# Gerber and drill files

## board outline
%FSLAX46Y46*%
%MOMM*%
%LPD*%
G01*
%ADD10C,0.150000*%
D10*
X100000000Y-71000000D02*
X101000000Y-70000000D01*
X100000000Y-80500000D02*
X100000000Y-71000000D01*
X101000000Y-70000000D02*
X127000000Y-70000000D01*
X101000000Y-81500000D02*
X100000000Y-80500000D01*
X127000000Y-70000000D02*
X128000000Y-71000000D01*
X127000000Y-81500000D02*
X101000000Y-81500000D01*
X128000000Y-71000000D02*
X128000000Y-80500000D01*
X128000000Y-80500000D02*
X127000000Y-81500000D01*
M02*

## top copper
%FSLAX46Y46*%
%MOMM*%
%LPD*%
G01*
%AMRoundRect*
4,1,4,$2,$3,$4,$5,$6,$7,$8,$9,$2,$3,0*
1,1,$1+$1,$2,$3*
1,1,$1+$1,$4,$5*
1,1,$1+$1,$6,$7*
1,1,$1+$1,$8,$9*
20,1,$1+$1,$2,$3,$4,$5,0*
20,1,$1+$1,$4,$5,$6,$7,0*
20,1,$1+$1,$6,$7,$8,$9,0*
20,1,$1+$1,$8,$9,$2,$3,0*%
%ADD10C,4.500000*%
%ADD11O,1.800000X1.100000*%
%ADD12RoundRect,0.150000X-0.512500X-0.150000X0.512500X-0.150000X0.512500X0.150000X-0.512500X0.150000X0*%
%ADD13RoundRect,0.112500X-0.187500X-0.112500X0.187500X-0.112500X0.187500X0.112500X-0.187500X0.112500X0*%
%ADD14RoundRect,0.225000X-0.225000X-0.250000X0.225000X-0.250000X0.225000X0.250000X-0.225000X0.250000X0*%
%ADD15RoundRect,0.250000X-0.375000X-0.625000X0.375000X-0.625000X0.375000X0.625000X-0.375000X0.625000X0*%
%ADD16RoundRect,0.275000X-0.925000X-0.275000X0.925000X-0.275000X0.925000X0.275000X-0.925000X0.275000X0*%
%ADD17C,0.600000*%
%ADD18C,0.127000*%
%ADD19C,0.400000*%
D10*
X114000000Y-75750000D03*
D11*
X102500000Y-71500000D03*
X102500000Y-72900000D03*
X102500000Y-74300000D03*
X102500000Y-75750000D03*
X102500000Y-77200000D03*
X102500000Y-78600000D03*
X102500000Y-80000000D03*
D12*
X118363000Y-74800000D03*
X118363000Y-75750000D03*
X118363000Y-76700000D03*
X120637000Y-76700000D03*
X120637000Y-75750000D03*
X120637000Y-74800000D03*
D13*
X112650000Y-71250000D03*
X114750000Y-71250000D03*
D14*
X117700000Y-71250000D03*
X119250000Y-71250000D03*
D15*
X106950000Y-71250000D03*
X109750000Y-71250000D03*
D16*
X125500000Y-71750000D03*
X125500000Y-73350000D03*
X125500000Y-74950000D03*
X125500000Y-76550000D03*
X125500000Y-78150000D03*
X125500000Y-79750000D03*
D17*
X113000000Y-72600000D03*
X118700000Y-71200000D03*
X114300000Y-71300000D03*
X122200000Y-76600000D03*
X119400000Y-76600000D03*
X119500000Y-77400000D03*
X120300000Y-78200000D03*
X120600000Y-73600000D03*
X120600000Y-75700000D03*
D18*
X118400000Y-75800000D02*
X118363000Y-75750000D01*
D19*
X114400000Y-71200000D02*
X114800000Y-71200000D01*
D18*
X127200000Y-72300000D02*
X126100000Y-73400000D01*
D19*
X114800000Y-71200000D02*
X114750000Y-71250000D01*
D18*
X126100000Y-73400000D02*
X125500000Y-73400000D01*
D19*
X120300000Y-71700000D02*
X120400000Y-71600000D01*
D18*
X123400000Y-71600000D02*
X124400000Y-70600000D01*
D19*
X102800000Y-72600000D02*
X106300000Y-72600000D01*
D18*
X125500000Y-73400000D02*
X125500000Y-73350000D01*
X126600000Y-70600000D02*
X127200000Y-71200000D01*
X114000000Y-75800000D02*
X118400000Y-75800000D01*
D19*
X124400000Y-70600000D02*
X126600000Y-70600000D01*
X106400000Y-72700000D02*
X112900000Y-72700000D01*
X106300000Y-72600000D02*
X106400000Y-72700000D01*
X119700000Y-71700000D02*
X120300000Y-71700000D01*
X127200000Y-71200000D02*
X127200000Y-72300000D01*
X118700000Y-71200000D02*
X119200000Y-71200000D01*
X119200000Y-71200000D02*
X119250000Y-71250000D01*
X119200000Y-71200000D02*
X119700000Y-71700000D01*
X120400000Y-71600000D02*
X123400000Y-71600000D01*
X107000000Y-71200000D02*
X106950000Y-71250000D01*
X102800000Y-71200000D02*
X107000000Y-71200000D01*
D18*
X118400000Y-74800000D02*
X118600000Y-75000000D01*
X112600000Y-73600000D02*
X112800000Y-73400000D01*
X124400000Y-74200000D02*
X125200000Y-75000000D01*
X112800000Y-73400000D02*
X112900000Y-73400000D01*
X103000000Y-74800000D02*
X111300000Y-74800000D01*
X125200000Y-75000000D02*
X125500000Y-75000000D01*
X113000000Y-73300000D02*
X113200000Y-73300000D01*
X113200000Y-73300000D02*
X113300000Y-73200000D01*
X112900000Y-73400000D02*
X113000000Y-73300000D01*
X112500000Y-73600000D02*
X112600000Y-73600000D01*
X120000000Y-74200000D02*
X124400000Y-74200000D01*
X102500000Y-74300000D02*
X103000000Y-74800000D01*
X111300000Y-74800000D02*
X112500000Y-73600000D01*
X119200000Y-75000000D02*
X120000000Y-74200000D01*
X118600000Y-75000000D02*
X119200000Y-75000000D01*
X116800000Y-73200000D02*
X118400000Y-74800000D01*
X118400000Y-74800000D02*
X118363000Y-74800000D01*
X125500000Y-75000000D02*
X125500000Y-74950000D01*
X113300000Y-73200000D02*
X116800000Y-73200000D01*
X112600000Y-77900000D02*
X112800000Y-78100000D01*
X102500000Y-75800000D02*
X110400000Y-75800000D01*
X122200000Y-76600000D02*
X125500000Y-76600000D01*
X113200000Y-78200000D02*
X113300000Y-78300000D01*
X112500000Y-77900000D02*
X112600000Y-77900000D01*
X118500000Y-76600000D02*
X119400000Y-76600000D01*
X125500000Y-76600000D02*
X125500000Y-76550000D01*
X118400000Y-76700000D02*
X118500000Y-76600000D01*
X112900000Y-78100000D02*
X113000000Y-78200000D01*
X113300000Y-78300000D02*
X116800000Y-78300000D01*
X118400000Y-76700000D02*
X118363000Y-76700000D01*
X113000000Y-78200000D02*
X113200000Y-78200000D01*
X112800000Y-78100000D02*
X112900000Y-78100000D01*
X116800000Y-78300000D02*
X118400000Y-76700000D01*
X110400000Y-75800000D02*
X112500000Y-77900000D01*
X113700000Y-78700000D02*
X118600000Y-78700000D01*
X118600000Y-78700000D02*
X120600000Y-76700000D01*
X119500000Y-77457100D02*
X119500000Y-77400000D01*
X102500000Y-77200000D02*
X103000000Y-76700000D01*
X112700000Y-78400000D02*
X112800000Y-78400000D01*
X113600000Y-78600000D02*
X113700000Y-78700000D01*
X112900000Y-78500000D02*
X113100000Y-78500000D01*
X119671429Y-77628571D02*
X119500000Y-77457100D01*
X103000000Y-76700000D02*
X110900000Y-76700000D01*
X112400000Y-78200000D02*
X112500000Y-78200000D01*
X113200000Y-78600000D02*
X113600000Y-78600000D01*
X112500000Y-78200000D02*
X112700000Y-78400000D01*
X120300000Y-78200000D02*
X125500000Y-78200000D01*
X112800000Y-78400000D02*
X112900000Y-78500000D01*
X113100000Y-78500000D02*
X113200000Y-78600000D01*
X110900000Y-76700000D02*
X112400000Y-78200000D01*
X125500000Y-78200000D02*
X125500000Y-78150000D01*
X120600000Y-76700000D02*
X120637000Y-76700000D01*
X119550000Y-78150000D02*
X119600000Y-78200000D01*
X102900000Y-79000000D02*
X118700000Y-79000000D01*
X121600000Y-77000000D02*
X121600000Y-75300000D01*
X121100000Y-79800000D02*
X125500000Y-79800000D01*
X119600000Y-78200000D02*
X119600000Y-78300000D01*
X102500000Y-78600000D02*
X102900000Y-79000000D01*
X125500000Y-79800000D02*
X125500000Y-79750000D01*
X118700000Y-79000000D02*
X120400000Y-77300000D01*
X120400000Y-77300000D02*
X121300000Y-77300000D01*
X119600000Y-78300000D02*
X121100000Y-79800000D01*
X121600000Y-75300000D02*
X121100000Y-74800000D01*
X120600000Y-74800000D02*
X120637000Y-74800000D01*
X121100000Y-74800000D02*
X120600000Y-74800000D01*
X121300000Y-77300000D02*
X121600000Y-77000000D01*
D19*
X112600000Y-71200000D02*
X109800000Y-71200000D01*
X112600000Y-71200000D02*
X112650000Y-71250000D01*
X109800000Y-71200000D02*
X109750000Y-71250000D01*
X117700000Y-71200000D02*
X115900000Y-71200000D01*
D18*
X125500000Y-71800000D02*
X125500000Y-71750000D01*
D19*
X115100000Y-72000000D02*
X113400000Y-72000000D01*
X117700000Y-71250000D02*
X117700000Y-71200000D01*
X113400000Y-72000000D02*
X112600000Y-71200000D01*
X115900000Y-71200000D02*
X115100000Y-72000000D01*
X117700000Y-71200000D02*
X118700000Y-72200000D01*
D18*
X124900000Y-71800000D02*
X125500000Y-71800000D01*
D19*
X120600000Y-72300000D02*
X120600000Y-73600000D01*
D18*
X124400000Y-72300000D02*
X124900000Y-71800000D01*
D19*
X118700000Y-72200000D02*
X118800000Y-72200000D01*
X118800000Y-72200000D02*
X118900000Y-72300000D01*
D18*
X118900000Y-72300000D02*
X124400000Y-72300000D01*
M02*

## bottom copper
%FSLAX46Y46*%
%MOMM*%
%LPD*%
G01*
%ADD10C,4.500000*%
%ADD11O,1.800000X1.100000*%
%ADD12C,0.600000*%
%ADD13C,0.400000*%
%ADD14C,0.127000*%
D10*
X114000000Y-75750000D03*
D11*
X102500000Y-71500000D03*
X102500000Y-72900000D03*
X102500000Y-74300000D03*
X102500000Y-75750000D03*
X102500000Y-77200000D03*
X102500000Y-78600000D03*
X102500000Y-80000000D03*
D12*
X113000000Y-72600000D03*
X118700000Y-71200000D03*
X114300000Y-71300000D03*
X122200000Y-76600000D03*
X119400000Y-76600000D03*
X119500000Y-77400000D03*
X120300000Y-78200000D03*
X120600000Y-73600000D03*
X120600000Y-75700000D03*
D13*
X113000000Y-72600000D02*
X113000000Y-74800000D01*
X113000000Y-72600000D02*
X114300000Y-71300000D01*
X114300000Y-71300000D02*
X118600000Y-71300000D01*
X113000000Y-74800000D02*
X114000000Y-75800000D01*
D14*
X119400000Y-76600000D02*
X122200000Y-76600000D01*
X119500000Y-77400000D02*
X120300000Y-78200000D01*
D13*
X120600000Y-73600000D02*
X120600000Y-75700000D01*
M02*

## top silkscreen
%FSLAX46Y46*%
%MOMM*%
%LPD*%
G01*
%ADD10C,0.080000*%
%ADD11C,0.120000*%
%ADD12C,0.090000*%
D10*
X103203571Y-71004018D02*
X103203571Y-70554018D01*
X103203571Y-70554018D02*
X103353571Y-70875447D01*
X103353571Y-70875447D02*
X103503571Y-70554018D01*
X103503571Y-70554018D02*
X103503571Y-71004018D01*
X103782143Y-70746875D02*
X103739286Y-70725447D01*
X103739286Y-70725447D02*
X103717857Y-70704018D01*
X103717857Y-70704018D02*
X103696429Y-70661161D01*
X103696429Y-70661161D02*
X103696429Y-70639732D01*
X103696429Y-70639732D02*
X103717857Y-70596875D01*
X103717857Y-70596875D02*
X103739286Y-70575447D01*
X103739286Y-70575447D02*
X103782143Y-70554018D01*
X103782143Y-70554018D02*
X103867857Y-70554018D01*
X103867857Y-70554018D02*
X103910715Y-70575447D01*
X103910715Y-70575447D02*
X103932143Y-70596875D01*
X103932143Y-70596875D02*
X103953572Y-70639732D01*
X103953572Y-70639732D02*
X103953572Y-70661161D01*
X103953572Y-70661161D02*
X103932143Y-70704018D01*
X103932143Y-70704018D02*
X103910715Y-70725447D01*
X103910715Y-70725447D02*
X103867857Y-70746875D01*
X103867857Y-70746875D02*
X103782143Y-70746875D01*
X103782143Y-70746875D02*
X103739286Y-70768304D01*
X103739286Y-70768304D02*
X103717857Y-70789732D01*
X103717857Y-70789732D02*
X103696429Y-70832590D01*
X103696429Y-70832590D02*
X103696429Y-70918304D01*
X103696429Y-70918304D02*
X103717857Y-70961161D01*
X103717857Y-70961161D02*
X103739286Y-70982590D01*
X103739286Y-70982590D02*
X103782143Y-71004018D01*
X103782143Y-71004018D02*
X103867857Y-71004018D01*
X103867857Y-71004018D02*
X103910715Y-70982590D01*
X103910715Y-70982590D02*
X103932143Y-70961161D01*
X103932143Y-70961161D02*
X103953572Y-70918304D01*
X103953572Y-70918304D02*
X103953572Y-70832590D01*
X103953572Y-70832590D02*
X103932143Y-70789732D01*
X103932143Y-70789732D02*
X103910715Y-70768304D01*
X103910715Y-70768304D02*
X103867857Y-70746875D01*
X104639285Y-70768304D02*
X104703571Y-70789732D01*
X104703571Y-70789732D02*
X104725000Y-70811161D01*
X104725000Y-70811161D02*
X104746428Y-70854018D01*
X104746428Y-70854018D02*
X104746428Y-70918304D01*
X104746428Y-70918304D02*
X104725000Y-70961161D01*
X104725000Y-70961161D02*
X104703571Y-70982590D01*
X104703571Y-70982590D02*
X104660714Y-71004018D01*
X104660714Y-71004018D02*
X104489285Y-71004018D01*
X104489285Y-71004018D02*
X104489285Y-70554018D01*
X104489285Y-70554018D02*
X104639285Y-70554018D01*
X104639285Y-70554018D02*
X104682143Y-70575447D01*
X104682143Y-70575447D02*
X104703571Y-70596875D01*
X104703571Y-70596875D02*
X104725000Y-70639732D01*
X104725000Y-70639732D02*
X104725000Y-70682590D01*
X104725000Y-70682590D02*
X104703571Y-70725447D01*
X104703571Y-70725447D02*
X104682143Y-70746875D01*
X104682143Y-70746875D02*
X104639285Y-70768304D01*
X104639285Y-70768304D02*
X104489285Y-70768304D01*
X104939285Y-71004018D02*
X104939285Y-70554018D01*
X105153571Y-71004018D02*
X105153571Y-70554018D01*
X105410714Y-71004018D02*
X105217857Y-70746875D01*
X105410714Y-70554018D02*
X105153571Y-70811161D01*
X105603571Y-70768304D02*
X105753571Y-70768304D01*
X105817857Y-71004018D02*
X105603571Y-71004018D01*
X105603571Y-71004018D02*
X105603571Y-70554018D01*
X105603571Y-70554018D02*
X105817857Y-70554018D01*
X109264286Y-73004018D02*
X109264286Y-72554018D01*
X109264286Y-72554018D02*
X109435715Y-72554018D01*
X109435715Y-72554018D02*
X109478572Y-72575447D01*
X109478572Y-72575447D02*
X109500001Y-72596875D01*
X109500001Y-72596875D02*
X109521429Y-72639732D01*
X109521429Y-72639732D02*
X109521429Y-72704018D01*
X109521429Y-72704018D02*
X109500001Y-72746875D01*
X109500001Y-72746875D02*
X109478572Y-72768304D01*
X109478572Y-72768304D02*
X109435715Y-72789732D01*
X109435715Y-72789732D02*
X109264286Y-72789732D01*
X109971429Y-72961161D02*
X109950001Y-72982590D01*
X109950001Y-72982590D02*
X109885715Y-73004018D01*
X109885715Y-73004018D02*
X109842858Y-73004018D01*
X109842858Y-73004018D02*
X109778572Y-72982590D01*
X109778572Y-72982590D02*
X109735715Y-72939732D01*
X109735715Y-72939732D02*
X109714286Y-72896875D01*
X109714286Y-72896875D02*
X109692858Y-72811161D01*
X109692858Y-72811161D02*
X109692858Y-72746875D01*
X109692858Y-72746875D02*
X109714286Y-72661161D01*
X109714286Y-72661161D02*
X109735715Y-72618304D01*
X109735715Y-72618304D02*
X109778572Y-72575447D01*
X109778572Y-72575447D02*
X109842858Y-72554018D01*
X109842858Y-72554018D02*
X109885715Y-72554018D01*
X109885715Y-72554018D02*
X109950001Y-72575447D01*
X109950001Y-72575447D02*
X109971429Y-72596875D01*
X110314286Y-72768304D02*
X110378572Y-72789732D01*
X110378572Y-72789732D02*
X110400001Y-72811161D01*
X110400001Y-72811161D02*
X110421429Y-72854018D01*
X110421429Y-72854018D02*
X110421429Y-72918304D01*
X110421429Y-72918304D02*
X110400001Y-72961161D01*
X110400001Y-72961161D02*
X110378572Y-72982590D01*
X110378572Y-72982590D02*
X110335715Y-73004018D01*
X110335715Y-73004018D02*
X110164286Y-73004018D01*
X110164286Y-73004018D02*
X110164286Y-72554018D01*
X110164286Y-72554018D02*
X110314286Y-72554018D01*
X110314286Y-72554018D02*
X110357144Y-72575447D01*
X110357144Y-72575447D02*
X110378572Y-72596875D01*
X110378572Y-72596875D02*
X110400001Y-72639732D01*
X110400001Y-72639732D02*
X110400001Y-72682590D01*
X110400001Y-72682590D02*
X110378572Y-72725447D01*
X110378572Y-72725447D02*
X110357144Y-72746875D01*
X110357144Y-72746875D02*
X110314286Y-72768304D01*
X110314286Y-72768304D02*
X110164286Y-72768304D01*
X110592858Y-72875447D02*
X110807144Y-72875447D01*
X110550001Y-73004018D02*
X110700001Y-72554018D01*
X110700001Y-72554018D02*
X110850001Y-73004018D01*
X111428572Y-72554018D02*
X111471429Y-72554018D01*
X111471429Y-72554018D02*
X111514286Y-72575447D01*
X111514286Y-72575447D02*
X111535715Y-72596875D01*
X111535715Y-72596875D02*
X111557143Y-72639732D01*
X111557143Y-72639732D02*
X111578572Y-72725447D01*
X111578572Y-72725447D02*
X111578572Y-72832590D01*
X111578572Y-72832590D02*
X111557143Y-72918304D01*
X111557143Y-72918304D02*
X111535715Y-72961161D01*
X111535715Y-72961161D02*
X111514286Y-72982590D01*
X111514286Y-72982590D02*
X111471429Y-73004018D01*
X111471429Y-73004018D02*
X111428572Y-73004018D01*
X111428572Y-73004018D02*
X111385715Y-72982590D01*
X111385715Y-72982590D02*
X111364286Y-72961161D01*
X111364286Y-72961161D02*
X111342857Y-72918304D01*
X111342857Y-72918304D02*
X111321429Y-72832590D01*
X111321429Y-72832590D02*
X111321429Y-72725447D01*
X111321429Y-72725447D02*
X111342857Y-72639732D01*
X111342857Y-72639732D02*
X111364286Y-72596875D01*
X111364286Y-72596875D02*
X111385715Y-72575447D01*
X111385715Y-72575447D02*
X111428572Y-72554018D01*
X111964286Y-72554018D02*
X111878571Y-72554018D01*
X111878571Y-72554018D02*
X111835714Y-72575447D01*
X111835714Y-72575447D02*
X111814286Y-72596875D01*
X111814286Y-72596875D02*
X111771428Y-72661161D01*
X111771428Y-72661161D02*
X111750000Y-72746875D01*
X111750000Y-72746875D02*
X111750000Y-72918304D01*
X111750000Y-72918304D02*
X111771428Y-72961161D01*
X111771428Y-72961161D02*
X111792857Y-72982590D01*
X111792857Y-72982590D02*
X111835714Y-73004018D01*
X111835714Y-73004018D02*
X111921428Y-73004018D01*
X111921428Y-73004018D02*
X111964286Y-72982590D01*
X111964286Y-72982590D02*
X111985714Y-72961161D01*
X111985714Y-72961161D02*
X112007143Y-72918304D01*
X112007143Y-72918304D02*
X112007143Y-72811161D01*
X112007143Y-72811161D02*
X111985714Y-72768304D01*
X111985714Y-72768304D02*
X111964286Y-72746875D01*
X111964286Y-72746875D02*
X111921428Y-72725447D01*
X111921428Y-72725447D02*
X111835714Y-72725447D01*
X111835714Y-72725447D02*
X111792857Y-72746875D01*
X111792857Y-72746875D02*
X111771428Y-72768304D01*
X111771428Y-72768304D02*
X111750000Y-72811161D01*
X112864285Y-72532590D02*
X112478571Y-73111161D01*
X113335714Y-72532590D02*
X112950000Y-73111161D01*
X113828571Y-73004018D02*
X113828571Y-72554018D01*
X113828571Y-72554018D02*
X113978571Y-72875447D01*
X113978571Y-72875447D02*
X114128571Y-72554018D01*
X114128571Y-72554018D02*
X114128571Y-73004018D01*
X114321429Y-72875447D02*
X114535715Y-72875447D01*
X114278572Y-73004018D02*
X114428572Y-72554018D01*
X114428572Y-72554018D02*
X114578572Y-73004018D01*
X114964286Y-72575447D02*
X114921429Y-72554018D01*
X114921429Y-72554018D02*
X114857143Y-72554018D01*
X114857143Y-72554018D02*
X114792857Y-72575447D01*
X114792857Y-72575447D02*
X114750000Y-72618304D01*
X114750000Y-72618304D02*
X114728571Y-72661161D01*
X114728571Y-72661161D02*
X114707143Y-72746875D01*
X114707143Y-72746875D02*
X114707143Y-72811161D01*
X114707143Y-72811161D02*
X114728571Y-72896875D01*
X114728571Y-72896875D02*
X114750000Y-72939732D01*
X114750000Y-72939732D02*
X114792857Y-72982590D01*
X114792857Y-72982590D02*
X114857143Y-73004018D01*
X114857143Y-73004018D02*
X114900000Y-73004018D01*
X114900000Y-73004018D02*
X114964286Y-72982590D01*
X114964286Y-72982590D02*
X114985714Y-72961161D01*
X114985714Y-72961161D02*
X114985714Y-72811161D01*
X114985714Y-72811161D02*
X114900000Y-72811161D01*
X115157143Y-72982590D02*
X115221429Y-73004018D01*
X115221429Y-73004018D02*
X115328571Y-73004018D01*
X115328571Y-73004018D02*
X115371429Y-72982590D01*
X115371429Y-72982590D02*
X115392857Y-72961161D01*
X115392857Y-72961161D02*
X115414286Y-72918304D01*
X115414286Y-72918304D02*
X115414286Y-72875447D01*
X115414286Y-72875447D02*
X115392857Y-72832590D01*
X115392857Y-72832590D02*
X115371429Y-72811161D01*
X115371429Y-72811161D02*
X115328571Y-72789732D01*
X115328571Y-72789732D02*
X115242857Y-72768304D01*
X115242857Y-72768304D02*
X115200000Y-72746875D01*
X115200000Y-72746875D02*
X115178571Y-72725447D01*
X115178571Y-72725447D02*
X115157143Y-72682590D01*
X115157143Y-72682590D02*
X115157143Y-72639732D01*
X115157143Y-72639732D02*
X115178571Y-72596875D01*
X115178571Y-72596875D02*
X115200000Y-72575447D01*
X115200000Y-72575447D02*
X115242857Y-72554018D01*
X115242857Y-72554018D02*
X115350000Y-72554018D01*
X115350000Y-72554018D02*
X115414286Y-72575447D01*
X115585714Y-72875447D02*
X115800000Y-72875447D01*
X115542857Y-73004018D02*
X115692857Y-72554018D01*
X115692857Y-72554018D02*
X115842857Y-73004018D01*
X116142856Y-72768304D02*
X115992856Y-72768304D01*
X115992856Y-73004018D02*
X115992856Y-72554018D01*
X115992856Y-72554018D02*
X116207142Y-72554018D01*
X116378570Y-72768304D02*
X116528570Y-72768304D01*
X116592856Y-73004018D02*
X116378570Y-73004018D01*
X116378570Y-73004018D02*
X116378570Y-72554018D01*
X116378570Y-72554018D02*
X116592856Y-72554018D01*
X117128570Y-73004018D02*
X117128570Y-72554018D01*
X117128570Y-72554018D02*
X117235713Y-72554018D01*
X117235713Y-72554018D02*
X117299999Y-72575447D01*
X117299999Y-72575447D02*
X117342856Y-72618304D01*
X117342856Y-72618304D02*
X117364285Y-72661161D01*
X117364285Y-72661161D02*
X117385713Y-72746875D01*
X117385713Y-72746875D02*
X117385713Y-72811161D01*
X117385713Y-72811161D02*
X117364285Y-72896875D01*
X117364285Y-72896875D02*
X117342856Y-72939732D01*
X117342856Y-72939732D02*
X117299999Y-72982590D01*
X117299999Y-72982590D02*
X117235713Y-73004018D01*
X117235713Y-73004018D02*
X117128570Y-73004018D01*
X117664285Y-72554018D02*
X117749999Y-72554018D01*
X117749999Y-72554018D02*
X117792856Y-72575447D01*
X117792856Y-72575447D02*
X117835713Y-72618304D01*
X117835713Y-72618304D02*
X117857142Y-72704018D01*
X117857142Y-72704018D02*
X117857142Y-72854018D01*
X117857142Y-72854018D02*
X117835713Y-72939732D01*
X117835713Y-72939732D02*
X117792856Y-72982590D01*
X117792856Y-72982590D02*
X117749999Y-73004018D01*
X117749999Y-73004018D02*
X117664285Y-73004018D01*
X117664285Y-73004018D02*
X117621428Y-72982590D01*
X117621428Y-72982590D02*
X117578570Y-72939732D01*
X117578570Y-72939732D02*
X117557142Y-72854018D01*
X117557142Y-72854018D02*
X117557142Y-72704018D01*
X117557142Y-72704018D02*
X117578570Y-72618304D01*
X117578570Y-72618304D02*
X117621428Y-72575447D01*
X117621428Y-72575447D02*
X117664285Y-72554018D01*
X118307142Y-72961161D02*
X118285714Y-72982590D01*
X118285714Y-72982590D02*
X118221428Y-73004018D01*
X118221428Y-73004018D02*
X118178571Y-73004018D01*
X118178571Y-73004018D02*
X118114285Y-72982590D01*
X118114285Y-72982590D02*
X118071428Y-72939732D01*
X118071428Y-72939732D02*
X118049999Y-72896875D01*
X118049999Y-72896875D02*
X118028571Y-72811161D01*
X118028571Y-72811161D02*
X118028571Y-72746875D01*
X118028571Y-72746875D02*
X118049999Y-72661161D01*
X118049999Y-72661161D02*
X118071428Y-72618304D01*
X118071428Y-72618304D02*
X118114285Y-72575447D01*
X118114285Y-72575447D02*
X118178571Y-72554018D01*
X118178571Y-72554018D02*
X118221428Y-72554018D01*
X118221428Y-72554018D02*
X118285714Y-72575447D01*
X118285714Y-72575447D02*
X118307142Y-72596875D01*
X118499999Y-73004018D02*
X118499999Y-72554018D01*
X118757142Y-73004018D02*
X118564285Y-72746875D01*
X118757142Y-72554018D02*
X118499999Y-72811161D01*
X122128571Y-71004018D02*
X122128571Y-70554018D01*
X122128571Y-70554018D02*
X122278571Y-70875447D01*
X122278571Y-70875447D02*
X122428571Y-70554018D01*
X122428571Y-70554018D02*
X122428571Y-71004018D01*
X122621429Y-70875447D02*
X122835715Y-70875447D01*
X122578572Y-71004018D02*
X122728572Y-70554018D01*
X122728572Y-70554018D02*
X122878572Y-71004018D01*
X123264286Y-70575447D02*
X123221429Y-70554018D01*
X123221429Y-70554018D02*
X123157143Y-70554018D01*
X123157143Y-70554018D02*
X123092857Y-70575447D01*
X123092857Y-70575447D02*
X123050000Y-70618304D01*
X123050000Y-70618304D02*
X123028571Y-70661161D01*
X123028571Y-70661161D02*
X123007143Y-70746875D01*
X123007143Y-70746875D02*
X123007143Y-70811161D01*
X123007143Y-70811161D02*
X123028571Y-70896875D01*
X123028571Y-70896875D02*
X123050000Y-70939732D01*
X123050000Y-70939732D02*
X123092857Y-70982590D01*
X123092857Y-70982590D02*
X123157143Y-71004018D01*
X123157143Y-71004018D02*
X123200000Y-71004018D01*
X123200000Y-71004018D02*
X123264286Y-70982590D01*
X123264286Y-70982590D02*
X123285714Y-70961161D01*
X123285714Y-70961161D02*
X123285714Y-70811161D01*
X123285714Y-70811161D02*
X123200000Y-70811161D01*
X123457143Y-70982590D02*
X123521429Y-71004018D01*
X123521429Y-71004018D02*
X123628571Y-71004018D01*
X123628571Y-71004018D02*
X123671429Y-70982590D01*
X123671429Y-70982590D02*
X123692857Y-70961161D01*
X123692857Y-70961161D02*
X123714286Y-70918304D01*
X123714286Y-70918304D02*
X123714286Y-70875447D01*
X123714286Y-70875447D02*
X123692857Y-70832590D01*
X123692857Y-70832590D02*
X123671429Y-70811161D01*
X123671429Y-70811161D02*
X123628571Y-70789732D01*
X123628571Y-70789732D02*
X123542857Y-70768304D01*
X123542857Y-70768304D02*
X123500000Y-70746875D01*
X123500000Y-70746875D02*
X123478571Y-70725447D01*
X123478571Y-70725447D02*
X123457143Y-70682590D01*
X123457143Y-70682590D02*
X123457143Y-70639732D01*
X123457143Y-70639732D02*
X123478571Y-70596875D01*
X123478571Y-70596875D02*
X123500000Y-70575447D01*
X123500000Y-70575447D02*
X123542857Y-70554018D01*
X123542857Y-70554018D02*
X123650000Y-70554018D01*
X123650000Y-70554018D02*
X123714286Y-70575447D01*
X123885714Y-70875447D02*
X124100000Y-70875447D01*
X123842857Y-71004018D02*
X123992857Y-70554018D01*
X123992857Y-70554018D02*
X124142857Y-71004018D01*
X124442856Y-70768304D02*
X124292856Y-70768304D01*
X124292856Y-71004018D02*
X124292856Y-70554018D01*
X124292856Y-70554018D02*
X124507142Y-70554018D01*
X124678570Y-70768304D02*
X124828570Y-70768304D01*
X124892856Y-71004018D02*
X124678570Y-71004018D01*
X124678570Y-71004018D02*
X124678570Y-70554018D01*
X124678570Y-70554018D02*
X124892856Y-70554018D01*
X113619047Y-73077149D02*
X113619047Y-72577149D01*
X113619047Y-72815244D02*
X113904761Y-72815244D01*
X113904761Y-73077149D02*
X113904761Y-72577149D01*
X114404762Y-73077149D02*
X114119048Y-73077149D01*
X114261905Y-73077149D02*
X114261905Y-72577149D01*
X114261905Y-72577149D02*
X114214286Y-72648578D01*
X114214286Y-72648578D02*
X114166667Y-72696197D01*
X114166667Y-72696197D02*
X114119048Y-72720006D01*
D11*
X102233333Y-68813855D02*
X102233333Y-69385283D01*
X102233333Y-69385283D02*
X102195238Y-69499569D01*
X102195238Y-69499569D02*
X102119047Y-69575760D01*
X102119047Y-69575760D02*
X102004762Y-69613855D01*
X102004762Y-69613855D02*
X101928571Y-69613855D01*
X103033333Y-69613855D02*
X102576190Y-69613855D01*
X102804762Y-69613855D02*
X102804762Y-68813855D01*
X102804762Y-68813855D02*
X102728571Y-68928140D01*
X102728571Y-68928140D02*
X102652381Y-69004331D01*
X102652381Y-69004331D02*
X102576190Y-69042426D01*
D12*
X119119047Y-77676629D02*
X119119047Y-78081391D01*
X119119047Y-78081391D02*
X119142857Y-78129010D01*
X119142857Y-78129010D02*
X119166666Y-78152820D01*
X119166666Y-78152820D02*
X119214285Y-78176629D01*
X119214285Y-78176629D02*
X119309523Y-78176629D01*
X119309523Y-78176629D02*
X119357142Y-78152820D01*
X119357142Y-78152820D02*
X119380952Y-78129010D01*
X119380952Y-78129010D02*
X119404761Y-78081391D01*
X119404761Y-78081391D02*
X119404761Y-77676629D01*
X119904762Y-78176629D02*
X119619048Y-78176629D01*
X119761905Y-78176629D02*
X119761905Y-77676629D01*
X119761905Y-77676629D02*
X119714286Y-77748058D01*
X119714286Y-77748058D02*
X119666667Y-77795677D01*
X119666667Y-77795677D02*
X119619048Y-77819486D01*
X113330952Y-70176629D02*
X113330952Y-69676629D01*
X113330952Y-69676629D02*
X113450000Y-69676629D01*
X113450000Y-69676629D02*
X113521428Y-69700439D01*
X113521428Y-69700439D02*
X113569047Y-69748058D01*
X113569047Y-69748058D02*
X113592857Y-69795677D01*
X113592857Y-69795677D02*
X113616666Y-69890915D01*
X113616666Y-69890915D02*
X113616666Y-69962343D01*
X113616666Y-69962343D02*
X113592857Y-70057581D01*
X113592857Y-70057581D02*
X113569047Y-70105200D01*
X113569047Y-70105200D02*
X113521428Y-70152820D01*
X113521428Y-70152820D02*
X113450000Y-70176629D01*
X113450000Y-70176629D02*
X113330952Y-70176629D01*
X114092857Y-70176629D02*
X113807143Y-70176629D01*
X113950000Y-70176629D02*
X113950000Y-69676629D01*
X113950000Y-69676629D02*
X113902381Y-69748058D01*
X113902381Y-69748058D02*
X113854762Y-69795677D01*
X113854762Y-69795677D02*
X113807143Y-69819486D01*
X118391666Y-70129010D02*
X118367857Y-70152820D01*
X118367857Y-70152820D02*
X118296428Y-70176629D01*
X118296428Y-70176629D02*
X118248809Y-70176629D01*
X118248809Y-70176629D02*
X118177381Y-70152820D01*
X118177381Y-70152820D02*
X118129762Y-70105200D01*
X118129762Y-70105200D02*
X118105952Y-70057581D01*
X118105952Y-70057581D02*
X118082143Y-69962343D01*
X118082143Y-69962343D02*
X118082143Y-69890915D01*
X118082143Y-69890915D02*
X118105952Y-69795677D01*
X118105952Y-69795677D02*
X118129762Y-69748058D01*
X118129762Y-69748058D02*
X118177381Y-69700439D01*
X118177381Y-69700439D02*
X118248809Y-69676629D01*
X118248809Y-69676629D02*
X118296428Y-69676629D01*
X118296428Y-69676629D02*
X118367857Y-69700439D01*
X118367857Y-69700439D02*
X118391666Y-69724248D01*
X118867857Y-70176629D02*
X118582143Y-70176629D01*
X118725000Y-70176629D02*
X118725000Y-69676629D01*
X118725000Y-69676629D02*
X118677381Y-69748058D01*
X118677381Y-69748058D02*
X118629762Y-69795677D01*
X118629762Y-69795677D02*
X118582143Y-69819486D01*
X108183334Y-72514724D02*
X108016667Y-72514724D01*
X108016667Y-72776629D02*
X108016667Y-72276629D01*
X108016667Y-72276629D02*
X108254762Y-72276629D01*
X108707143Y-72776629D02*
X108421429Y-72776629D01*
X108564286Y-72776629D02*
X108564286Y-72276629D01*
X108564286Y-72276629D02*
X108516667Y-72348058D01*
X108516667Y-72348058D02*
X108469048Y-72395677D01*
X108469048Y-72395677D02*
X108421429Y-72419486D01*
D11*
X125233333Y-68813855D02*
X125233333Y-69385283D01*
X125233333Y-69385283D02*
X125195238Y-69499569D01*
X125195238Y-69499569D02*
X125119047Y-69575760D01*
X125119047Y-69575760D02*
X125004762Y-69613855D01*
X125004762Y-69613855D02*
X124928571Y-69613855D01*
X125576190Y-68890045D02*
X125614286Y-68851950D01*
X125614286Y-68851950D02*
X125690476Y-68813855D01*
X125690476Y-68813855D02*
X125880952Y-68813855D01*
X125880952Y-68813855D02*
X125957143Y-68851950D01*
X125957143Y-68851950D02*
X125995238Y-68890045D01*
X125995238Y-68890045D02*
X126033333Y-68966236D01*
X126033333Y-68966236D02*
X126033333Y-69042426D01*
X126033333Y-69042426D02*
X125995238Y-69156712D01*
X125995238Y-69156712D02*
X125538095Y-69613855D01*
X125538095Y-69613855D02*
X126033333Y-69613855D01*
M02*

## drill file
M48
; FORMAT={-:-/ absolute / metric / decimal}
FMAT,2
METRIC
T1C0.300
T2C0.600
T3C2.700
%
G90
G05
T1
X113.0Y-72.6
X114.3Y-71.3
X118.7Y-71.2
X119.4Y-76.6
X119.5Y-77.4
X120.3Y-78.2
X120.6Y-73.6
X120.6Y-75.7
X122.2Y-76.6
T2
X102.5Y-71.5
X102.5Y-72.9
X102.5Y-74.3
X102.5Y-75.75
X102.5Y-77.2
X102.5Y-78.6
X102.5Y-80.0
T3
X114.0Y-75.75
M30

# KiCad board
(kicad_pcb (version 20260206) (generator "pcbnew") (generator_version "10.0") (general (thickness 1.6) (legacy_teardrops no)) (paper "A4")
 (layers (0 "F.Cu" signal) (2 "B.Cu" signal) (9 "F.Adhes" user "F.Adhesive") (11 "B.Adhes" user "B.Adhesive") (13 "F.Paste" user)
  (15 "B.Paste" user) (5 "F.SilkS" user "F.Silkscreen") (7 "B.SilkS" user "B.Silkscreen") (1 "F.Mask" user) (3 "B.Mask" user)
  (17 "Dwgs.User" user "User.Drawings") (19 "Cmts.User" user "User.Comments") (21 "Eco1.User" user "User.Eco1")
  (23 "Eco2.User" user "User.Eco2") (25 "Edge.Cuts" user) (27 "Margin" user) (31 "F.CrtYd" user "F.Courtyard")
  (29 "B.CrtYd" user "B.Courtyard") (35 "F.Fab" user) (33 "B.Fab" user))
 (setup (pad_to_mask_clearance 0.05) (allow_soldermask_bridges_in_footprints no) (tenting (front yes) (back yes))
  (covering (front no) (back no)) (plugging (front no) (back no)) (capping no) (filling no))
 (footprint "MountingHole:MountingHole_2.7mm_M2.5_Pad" (layer "F.Cu") (at 114 75.75)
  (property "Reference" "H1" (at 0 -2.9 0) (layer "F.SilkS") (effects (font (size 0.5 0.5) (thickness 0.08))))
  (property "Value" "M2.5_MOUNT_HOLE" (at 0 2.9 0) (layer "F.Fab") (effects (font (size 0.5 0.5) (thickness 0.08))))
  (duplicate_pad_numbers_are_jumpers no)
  (pad "1" thru_hole circle (at 0 0) (size 4.5 4.5) (drill 2.7) (layers "*.Cu" "*.Mask") (remove_unused_layers no) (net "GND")))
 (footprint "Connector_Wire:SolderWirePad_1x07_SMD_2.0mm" (layer "F.Cu") (at 102.5 75.75)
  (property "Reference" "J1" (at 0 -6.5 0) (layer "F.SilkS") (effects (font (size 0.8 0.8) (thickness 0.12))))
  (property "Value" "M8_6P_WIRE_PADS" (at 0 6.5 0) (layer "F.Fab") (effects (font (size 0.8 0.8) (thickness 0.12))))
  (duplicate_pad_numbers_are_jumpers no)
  (pad "1" thru_hole oval (at 0 -4.25) (size 1.8 1.1) (drill 0.6) (layers "*.Cu" "*.Mask") (remove_unused_layers no) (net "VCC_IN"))
  (pad "2" thru_hole oval (at 0 -2.85) (size 1.8 1.1) (drill 0.6) (layers "*.Cu" "*.Mask") (remove_unused_layers no) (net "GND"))
  (pad "3" thru_hole oval (at 0 -1.45) (size 1.8 1.1) (drill 0.6) (layers "*.Cu" "*.Mask") (remove_unused_layers no) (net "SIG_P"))
  (pad "4" thru_hole oval (at 0 0) (size 1.8 1.1) (drill 0.6) (layers "*.Cu" "*.Mask") (remove_unused_layers no) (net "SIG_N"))
  (pad "5" thru_hole oval (at 0 1.45) (size 1.8 1.1) (drill 0.6) (layers "*.Cu" "*.Mask") (remove_unused_layers no) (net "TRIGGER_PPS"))
  (pad "6" thru_hole oval (at 0 2.85) (size 1.8 1.1) (drill 0.6) (layers "*.Cu" "*.Mask") (remove_unused_layers no) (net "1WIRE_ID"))
  (pad "7" thru_hole oval (at 0 4.25) (size 1.8 1.1) (drill 0.6) (layers "*.Cu" "*.Mask") (remove_unused_layers no) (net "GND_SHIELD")))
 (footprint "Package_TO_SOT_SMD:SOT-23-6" (layer "F.Cu") (at 119.5 75.75)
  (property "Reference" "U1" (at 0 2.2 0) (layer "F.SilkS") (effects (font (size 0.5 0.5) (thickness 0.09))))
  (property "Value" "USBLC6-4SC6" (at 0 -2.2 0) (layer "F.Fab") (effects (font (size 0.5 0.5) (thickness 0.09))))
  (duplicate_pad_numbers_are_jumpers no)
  (pad "1" smd roundrect (at -1.137 -0.95) (size 1.325 0.6) (layers "F.Cu" "F.Mask" "F.Paste") (roundrect_rratio 0.25) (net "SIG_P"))
  (pad "2" smd roundrect (at -1.137 0) (size 1.325 0.6) (layers "F.Cu" "F.Mask" "F.Paste") (roundrect_rratio 0.25) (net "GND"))
  (pad "3" smd roundrect (at -1.137 0.95) (size 1.325 0.6) (layers "F.Cu" "F.Mask" "F.Paste") (roundrect_rratio 0.25) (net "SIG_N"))
  (pad "4" smd roundrect (at 1.137 0.95) (size 1.325 0.6) (layers "F.Cu" "F.Mask" "F.Paste") (roundrect_rratio 0.25) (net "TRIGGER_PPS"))
  (pad "5" smd roundrect (at 1.137 0) (size 1.325 0.6) (layers "F.Cu" "F.Mask" "F.Paste") (roundrect_rratio 0.25) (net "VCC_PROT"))
  (pad "6" smd roundrect (at 1.137 -0.95) (size 1.325 0.6) (layers "F.Cu" "F.Mask" "F.Paste") (roundrect_rratio 0.25) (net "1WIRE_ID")))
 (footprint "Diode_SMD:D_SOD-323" (layer "F.Cu") (at 113.7 71.25)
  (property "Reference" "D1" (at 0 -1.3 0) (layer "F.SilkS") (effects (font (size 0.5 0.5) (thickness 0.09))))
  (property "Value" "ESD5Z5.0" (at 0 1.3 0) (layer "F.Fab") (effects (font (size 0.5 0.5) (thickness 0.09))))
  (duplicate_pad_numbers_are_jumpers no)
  (pad "1" smd roundrect (at -1.05 0) (size 0.6 0.45) (layers "F.Cu" "F.Mask" "F.Paste") (roundrect_rratio 0.25) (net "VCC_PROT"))
  (pad "2" smd roundrect (at 1.05 0) (size 0.6 0.45) (layers "F.Cu" "F.Mask" "F.Paste") (roundrect_rratio 0.25) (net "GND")))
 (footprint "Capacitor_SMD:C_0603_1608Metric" (layer "F.Cu") (at 118.475 71.25)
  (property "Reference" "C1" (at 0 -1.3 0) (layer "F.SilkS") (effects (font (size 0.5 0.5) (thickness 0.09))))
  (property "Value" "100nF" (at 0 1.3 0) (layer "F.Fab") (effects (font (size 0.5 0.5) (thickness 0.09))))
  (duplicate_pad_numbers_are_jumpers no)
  (pad "1" smd roundrect (at -0.775 0) (size 0.9 0.95) (layers "F.Cu" "F.Mask" "F.Paste") (roundrect_rratio 0.25) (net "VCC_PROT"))
  (pad "2" smd roundrect (at 0.775 0) (size 0.9 0.95) (layers "F.Cu" "F.Mask" "F.Paste") (roundrect_rratio 0.25) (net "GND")))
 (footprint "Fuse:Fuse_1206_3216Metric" (layer "F.Cu") (at 108.35 71.25)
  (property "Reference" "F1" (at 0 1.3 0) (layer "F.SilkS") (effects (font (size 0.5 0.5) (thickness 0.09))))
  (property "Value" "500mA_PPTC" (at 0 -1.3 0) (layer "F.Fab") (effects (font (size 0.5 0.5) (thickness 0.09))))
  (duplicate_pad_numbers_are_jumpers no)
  (pad "1" smd roundrect (at -1.4 0) (size 1.25 1.75) (layers "F.Cu" "F.Mask" "F.Paste") (roundrect_rratio 0.2) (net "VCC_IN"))
  (pad "2" smd roundrect (at 1.4 0) (size 1.25 1.75) (layers "F.Cu" "F.Mask" "F.Paste") (roundrect_rratio 0.2) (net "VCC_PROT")))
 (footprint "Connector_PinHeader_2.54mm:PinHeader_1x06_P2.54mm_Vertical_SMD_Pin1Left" (layer "F.Cu") (at 125.5 75.75)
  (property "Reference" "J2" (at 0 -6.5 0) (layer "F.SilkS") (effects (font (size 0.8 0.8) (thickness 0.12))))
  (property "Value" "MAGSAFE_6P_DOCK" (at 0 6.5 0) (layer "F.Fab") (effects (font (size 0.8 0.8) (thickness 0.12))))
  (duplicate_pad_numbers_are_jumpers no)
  (pad "1" smd roundrect (at 0 -4) (size 2.4 1.1) (layers "F.Cu" "F.Mask" "F.Paste") (roundrect_rratio 0.25) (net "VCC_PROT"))
  (pad "2" smd roundrect (at 0 -2.4) (size 2.4 1.1) (layers "F.Cu" "F.Mask" "F.Paste") (roundrect_rratio 0.25) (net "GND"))
  (pad "3" smd roundrect (at 0 -0.8) (size 2.4 1.1) (layers "F.Cu" "F.Mask" "F.Paste") (roundrect_rratio 0.25) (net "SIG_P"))
  (pad "4" smd roundrect (at 0 0.8) (size 2.4 1.1) (layers "F.Cu" "F.Mask" "F.Paste") (roundrect_rratio 0.25) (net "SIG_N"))
  (pad "5" smd roundrect (at 0 2.4) (size 2.4 1.1) (layers "F.Cu" "F.Mask" "F.Paste") (roundrect_rratio 0.25) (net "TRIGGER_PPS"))
  (pad "6" smd roundrect (at 0 4) (size 2.4 1.1) (layers "F.Cu" "F.Mask" "F.Paste") (roundrect_rratio 0.25) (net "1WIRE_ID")))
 (gr_line (start 100 71) (end 101 70) (stroke (width 0.15) (type solid)) (layer "Edge.Cuts"))
 (gr_line (start 100 80.5) (end 100 71) (stroke (width 0.15) (type solid)) (layer "Edge.Cuts"))
 (gr_line (start 101 70) (end 127 70) (stroke (width 0.15) (type solid)) (layer "Edge.Cuts"))
 (gr_line (start 101 81.5) (end 100 80.5) (stroke (width 0.15) (type solid)) (layer "Edge.Cuts"))
 (gr_line (start 127 70) (end 128 71) (stroke (width 0.15) (type solid)) (layer "Edge.Cuts"))
 (gr_line (start 127 81.5) (end 101 81.5) (stroke (width 0.15) (type solid)) (layer "Edge.Cuts"))
 (gr_line (start 128 71) (end 128 80.5) (stroke (width 0.15) (type solid)) (layer "Edge.Cuts"))
 (gr_line (start 128 80.5) (end 127 81.5) (stroke (width 0.15) (type solid)) (layer "Edge.Cuts"))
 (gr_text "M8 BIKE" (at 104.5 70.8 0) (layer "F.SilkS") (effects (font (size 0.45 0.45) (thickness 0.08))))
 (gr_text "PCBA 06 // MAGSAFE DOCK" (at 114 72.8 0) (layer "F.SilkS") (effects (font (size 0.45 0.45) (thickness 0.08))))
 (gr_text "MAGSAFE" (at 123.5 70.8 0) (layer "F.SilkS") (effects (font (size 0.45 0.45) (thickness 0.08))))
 (segment (start 118.4 75.8) (end 118.363 75.75) (width 0.127) (layer "F.Cu") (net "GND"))
 (segment (start 114.4 71.2) (end 114.8 71.2) (width 0.4) (layer "F.Cu") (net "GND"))
 (segment (start 127.2 72.3) (end 126.1 73.4) (width 0.127) (layer "F.Cu") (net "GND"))
 (segment (start 114.8 71.2) (end 114.75 71.25) (width 0.4) (layer "F.Cu") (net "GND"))
 (segment (start 126.1 73.4) (end 125.5 73.4) (width 0.127) (layer "F.Cu") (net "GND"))
 (segment (start 120.3 71.7) (end 120.4 71.6) (width 0.4) (layer "F.Cu") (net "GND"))
 (segment (start 123.4 71.6) (end 124.4 70.6) (width 0.127) (layer "F.Cu") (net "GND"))
 (segment (start 102.8 72.6) (end 106.3 72.6) (width 0.4) (layer "F.Cu") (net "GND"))
 (segment (start 125.5 73.4) (end 125.5 73.35) (width 0.127) (layer "F.Cu") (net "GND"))
 (segment (start 126.6 70.6) (end 127.2 71.2) (width 0.127) (layer "F.Cu") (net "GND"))
 (segment (start 114 75.8) (end 118.4 75.8) (width 0.127) (layer "F.Cu") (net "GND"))
 (segment (start 124.4 70.6) (end 126.6 70.6) (width 0.4) (layer "F.Cu") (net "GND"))
 (segment (start 106.4 72.7) (end 112.9 72.7) (width 0.4) (layer "F.Cu") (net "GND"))
 (segment (start 106.3 72.6) (end 106.4 72.7) (width 0.4) (layer "F.Cu") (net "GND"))
 (segment (start 119.7 71.7) (end 120.3 71.7) (width 0.4) (layer "F.Cu") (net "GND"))
 (segment (start 127.2 71.2) (end 127.2 72.3) (width 0.4) (layer "F.Cu") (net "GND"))
 (segment (start 118.7 71.2) (end 119.2 71.2) (width 0.4) (layer "F.Cu") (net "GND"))
 (segment (start 119.2 71.2) (end 119.25 71.25) (width 0.4) (layer "F.Cu") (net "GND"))
 (segment (start 119.2 71.2) (end 119.7 71.7) (width 0.4) (layer "F.Cu") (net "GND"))
 (segment (start 120.4 71.6) (end 123.4 71.6) (width 0.4) (layer "F.Cu") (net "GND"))
 (via (at 113 72.6) (size 0.6) (drill 0.3) (layers "F.Cu" "B.Cu") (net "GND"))
 (via (at 118.7 71.2) (size 0.6) (drill 0.3) (layers "F.Cu" "B.Cu") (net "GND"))
 (via (at 114.3 71.3) (size 0.6) (drill 0.3) (layers "F.Cu" "B.Cu") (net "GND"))
 (segment (start 113 72.6) (end 113 74.8) (width 0.4) (layer "B.Cu") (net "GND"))
 (segment (start 113 72.6) (end 114.3 71.3) (width 0.4) (layer "B.Cu") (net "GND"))
 (segment (start 114.3 71.3) (end 118.6 71.3) (width 0.4) (layer "B.Cu") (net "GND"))
 (segment (start 113 74.8) (end 114 75.8) (width 0.4) (layer "B.Cu") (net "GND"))
 (segment (start 107 71.2) (end 106.95 71.25) (width 0.4) (layer "F.Cu") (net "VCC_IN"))
 (segment (start 102.8 71.2) (end 107 71.2) (width 0.4) (layer "F.Cu") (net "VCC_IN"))
 (segment (start 118.4 74.8) (end 118.6 75) (width 0.127) (layer "F.Cu") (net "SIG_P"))
 (segment (start 112.6 73.6) (end 112.8 73.4) (width 0.127) (layer "F.Cu") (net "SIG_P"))
 (segment (start 124.4 74.2) (end 125.2 75) (width 0.127) (layer "F.Cu") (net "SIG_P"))
 (segment (start 112.8 73.4) (end 112.9 73.4) (width 0.127) (layer "F.Cu") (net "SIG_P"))
 (segment (start 103 74.8) (end 111.3 74.8) (width 0.127) (layer "F.Cu") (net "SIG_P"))
 (segment (start 125.2 75) (end 125.5 75) (width 0.127) (layer "F.Cu") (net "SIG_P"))
 (segment (start 113 73.3) (end 113.2 73.3) (width 0.127) (layer "F.Cu") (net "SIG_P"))
 (segment (start 113.2 73.3) (end 113.3 73.2) (width 0.127) (layer "F.Cu") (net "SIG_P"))
 (segment (start 112.9 73.4) (end 113 73.3) (width 0.127) (layer "F.Cu") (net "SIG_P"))
 (segment (start 112.5 73.6) (end 112.6 73.6) (width 0.127) (layer "F.Cu") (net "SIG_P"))
 (segment (start 120 74.2) (end 124.4 74.2) (width 0.127) (layer "F.Cu") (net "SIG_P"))
 (segment (start 102.5 74.3) (end 103 74.8) (width 0.127) (layer "F.Cu") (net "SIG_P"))
 (segment (start 111.3 74.8) (end 112.5 73.6) (width 0.127) (layer "F.Cu") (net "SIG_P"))
 (segment (start 119.2 75) (end 120 74.2) (width 0.127) (layer "F.Cu") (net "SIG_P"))
 (segment (start 118.6 75) (end 119.2 75) (width 0.127) (layer "F.Cu") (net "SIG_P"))
 (segment (start 116.8 73.2) (end 118.4 74.8) (width 0.127) (layer "F.Cu") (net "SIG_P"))
 (segment (start 118.4 74.8) (end 118.363 74.8) (width 0.127) (layer "F.Cu") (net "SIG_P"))
 (segment (start 125.5 75) (end 125.5 74.95) (width 0.127) (layer "F.Cu") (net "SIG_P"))
 (segment (start 113.3 73.2) (end 116.8 73.2) (width 0.127) (layer "F.Cu") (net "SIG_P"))
 (segment (start 112.6 77.9) (end 112.8 78.1) (width 0.127) (layer "F.Cu") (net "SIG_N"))
 (segment (start 102.5 75.8) (end 110.4 75.8) (width 0.127) (layer "F.Cu") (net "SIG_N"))
 (segment (start 122.2 76.6) (end 125.5 76.6) (width 0.127) (layer "F.Cu") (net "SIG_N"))
 (segment (start 113.2 78.2) (end 113.3 78.3) (width 0.127) (layer "F.Cu") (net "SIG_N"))
 (segment (start 112.5 77.9) (end 112.6 77.9) (width 0.127) (layer "F.Cu") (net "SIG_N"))
 (segment (start 118.5 76.6) (end 119.4 76.6) (width 0.127) (layer "F.Cu") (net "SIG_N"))
 (segment (start 125.5 76.6) (end 125.5 76.55) (width 0.127) (layer "F.Cu") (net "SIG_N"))
 (segment (start 118.4 76.7) (end 118.5 76.6) (width 0.127) (layer "F.Cu") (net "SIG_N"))
 (segment (start 112.9 78.1) (end 113 78.2) (width 0.127) (layer "F.Cu") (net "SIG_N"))
 (segment (start 113.3 78.3) (end 116.8 78.3) (width 0.127) (layer "F.Cu") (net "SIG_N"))
 (segment (start 118.4 76.7) (end 118.363 76.7) (width 0.127) (layer "F.Cu") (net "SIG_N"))
 (segment (start 113 78.2) (end 113.2 78.2) (width 0.127) (layer "F.Cu") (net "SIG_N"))
 (segment (start 112.8 78.1) (end 112.9 78.1) (width 0.127) (layer "F.Cu") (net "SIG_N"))
 (segment (start 116.8 78.3) (end 118.4 76.7) (width 0.127) (layer "F.Cu") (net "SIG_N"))
 (segment (start 110.4 75.8) (end 112.5 77.9) (width 0.127) (layer "F.Cu") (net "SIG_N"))
 (via (at 122.2 76.6) (size 0.6) (drill 0.3) (layers "F.Cu" "B.Cu") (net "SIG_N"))
 (via (at 119.4 76.6) (size 0.6) (drill 0.3) (layers "F.Cu" "B.Cu") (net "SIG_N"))
 (segment (start 119.4 76.6) (end 122.2 76.6) (width 0.127) (layer "B.Cu") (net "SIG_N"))
 (segment (start 113.7 78.7) (end 118.6 78.7) (width 0.127) (layer "F.Cu") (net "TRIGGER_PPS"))
 (segment (start 118.6 78.7) (end 120.6 76.7) (width 0.127) (layer "F.Cu") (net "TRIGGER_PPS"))
 (segment (start 119.5 77.4571) (end 119.5 77.4) (width 0.127) (layer "F.Cu") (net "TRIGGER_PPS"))
 (segment (start 102.5 77.2) (end 103 76.7) (width 0.127) (layer "F.Cu") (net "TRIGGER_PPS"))
 (segment (start 112.7 78.4) (end 112.8 78.4) (width 0.127) (layer "F.Cu") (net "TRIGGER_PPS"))
 (segment (start 113.6 78.6) (end 113.7 78.7) (width 0.127) (layer "F.Cu") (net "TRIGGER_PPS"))
 (segment (start 112.9 78.5) (end 113.1 78.5) (width 0.127) (layer "F.Cu") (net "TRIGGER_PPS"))
 (segment (start 119.671429 77.628571) (end 119.5 77.4571) (width 0.127) (layer "F.Cu") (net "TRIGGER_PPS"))
 (segment (start 103 76.7) (end 110.9 76.7) (width 0.127) (layer "F.Cu") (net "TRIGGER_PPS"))
 (segment (start 112.4 78.2) (end 112.5 78.2) (width 0.127) (layer "F.Cu") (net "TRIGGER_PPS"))
 (segment (start 113.2 78.6) (end 113.6 78.6) (width 0.127) (layer "F.Cu") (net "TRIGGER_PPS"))
 (segment (start 112.5 78.2) (end 112.7 78.4) (width 0.127) (layer "F.Cu") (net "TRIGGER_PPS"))
 (segment (start 120.3 78.2) (end 125.5 78.2) (width 0.127) (layer "F.Cu") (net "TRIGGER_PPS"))
 (segment (start 112.8 78.4) (end 112.9 78.5) (width 0.127) (layer "F.Cu") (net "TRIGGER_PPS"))
 (segment (start 113.1 78.5) (end 113.2 78.6) (width 0.127) (layer "F.Cu") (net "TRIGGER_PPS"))
 (segment (start 110.9 76.7) (end 112.4 78.2) (width 0.127) (layer "F.Cu") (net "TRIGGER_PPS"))
 (segment (start 125.5 78.2) (end 125.5 78.15) (width 0.127) (layer "F.Cu") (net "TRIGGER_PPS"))
 (segment (start 120.6 76.7) (end 120.637 76.7) (width 0.127) (layer "F.Cu") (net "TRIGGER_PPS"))
 (via (at 119.5 77.4) (size 0.6) (drill 0.3) (layers "F.Cu" "B.Cu") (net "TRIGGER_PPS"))
 (via (at 120.3 78.2) (size 0.6) (drill 0.3) (layers "F.Cu" "B.Cu") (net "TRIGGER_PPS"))
 (segment (start 119.5 77.4) (end 120.3 78.2) (width 0.127) (layer "B.Cu") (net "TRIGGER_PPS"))
 (segment (start 119.55 78.15) (end 119.6 78.2) (width 0.127) (layer "F.Cu") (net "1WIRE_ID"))
 (segment (start 102.9 79) (end 118.7 79) (width 0.127) (layer "F.Cu") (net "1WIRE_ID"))
 (segment (start 121.6 77) (end 121.6 75.3) (width 0.127) (layer "F.Cu") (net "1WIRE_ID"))
 (segment (start 121.1 79.8) (end 125.5 79.8) (width 0.127) (layer "F.Cu") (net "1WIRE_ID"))
 (segment (start 119.6 78.2) (end 119.6 78.3) (width 0.127) (layer "F.Cu") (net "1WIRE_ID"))
 (segment (start 102.5 78.6) (end 102.9 79) (width 0.127) (layer "F.Cu") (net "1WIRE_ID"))
 (segment (start 125.5 79.8) (end 125.5 79.75) (width 0.127) (layer "F.Cu") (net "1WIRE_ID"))
 (segment (start 118.7 79) (end 120.4 77.3) (width 0.127) (layer "F.Cu") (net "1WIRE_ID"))
 (segment (start 120.4 77.3) (end 121.3 77.3) (width 0.127) (layer "F.Cu") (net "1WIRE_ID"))
 (segment (start 119.6 78.3) (end 121.1 79.8) (width 0.127) (layer "F.Cu") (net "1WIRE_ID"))
 (segment (start 121.6 75.3) (end 121.1 74.8) (width 0.127) (layer "F.Cu") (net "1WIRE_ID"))
 (segment (start 120.6 74.8) (end 120.637 74.8) (width 0.127) (layer "F.Cu") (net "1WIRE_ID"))
 (segment (start 121.1 74.8) (end 120.6 74.8) (width 0.127) (layer "F.Cu") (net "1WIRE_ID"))
 (segment (start 121.3 77.3) (end 121.6 77) (width 0.127) (layer "F.Cu") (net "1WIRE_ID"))
 (segment (start 112.6 71.2) (end 109.8 71.2) (width 0.4) (layer "F.Cu") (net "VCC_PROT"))
 (segment (start 112.6 71.2) (end 112.65 71.25) (width 0.4) (layer "F.Cu") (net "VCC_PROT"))
 (segment (start 109.8 71.2) (end 109.75 71.25) (width 0.4) (layer "F.Cu") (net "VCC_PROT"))
 (segment (start 117.7 71.2) (end 115.9 71.2) (width 0.4) (layer "F.Cu") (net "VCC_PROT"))
 (segment (start 125.5 71.8) (end 125.5 71.75) (width 0.127) (layer "F.Cu") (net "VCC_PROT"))
 (segment (start 115.1 72) (end 113.4 72) (width 0.4) (layer "F.Cu") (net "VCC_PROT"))
 (segment (start 117.7 71.25) (end 117.7 71.2) (width 0.4) (layer "F.Cu") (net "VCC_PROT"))
 (segment (start 113.4 72) (end 112.6 71.2) (width 0.4) (layer "F.Cu") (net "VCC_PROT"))
 (segment (start 115.9 71.2) (end 115.1 72) (width 0.4) (layer "F.Cu") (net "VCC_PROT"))
 (segment (start 117.7 71.2) (end 118.7 72.2) (width 0.4) (layer "F.Cu") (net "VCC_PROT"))
 (segment (start 124.9 71.8) (end 125.5 71.8) (width 0.127) (layer "F.Cu") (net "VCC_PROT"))
 (segment (start 120.6 72.3) (end 120.6 73.6) (width 0.4) (layer "F.Cu") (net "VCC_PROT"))
 (segment (start 124.4 72.3) (end 124.9 71.8) (width 0.127) (layer "F.Cu") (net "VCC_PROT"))
 (segment (start 118.7 72.2) (end 118.8 72.2) (width 0.4) (layer "F.Cu") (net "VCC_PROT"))
 (segment (start 118.8 72.2) (end 118.9 72.3) (width 0.4) (layer "F.Cu") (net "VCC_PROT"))
 (segment (start 118.9 72.3) (end 124.4 72.3) (width 0.127) (layer "F.Cu") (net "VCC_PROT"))
 (via (at 120.6 73.6) (size 0.6) (drill 0.3) (layers "F.Cu" "B.Cu") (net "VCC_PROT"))
 (via (at 120.6 75.7) (size 0.6) (drill 0.3) (layers "F.Cu" "B.Cu") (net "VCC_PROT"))
 (segment (start 120.6 73.6) (end 120.6 75.7) (width 0.4) (layer "B.Cu") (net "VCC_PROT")))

